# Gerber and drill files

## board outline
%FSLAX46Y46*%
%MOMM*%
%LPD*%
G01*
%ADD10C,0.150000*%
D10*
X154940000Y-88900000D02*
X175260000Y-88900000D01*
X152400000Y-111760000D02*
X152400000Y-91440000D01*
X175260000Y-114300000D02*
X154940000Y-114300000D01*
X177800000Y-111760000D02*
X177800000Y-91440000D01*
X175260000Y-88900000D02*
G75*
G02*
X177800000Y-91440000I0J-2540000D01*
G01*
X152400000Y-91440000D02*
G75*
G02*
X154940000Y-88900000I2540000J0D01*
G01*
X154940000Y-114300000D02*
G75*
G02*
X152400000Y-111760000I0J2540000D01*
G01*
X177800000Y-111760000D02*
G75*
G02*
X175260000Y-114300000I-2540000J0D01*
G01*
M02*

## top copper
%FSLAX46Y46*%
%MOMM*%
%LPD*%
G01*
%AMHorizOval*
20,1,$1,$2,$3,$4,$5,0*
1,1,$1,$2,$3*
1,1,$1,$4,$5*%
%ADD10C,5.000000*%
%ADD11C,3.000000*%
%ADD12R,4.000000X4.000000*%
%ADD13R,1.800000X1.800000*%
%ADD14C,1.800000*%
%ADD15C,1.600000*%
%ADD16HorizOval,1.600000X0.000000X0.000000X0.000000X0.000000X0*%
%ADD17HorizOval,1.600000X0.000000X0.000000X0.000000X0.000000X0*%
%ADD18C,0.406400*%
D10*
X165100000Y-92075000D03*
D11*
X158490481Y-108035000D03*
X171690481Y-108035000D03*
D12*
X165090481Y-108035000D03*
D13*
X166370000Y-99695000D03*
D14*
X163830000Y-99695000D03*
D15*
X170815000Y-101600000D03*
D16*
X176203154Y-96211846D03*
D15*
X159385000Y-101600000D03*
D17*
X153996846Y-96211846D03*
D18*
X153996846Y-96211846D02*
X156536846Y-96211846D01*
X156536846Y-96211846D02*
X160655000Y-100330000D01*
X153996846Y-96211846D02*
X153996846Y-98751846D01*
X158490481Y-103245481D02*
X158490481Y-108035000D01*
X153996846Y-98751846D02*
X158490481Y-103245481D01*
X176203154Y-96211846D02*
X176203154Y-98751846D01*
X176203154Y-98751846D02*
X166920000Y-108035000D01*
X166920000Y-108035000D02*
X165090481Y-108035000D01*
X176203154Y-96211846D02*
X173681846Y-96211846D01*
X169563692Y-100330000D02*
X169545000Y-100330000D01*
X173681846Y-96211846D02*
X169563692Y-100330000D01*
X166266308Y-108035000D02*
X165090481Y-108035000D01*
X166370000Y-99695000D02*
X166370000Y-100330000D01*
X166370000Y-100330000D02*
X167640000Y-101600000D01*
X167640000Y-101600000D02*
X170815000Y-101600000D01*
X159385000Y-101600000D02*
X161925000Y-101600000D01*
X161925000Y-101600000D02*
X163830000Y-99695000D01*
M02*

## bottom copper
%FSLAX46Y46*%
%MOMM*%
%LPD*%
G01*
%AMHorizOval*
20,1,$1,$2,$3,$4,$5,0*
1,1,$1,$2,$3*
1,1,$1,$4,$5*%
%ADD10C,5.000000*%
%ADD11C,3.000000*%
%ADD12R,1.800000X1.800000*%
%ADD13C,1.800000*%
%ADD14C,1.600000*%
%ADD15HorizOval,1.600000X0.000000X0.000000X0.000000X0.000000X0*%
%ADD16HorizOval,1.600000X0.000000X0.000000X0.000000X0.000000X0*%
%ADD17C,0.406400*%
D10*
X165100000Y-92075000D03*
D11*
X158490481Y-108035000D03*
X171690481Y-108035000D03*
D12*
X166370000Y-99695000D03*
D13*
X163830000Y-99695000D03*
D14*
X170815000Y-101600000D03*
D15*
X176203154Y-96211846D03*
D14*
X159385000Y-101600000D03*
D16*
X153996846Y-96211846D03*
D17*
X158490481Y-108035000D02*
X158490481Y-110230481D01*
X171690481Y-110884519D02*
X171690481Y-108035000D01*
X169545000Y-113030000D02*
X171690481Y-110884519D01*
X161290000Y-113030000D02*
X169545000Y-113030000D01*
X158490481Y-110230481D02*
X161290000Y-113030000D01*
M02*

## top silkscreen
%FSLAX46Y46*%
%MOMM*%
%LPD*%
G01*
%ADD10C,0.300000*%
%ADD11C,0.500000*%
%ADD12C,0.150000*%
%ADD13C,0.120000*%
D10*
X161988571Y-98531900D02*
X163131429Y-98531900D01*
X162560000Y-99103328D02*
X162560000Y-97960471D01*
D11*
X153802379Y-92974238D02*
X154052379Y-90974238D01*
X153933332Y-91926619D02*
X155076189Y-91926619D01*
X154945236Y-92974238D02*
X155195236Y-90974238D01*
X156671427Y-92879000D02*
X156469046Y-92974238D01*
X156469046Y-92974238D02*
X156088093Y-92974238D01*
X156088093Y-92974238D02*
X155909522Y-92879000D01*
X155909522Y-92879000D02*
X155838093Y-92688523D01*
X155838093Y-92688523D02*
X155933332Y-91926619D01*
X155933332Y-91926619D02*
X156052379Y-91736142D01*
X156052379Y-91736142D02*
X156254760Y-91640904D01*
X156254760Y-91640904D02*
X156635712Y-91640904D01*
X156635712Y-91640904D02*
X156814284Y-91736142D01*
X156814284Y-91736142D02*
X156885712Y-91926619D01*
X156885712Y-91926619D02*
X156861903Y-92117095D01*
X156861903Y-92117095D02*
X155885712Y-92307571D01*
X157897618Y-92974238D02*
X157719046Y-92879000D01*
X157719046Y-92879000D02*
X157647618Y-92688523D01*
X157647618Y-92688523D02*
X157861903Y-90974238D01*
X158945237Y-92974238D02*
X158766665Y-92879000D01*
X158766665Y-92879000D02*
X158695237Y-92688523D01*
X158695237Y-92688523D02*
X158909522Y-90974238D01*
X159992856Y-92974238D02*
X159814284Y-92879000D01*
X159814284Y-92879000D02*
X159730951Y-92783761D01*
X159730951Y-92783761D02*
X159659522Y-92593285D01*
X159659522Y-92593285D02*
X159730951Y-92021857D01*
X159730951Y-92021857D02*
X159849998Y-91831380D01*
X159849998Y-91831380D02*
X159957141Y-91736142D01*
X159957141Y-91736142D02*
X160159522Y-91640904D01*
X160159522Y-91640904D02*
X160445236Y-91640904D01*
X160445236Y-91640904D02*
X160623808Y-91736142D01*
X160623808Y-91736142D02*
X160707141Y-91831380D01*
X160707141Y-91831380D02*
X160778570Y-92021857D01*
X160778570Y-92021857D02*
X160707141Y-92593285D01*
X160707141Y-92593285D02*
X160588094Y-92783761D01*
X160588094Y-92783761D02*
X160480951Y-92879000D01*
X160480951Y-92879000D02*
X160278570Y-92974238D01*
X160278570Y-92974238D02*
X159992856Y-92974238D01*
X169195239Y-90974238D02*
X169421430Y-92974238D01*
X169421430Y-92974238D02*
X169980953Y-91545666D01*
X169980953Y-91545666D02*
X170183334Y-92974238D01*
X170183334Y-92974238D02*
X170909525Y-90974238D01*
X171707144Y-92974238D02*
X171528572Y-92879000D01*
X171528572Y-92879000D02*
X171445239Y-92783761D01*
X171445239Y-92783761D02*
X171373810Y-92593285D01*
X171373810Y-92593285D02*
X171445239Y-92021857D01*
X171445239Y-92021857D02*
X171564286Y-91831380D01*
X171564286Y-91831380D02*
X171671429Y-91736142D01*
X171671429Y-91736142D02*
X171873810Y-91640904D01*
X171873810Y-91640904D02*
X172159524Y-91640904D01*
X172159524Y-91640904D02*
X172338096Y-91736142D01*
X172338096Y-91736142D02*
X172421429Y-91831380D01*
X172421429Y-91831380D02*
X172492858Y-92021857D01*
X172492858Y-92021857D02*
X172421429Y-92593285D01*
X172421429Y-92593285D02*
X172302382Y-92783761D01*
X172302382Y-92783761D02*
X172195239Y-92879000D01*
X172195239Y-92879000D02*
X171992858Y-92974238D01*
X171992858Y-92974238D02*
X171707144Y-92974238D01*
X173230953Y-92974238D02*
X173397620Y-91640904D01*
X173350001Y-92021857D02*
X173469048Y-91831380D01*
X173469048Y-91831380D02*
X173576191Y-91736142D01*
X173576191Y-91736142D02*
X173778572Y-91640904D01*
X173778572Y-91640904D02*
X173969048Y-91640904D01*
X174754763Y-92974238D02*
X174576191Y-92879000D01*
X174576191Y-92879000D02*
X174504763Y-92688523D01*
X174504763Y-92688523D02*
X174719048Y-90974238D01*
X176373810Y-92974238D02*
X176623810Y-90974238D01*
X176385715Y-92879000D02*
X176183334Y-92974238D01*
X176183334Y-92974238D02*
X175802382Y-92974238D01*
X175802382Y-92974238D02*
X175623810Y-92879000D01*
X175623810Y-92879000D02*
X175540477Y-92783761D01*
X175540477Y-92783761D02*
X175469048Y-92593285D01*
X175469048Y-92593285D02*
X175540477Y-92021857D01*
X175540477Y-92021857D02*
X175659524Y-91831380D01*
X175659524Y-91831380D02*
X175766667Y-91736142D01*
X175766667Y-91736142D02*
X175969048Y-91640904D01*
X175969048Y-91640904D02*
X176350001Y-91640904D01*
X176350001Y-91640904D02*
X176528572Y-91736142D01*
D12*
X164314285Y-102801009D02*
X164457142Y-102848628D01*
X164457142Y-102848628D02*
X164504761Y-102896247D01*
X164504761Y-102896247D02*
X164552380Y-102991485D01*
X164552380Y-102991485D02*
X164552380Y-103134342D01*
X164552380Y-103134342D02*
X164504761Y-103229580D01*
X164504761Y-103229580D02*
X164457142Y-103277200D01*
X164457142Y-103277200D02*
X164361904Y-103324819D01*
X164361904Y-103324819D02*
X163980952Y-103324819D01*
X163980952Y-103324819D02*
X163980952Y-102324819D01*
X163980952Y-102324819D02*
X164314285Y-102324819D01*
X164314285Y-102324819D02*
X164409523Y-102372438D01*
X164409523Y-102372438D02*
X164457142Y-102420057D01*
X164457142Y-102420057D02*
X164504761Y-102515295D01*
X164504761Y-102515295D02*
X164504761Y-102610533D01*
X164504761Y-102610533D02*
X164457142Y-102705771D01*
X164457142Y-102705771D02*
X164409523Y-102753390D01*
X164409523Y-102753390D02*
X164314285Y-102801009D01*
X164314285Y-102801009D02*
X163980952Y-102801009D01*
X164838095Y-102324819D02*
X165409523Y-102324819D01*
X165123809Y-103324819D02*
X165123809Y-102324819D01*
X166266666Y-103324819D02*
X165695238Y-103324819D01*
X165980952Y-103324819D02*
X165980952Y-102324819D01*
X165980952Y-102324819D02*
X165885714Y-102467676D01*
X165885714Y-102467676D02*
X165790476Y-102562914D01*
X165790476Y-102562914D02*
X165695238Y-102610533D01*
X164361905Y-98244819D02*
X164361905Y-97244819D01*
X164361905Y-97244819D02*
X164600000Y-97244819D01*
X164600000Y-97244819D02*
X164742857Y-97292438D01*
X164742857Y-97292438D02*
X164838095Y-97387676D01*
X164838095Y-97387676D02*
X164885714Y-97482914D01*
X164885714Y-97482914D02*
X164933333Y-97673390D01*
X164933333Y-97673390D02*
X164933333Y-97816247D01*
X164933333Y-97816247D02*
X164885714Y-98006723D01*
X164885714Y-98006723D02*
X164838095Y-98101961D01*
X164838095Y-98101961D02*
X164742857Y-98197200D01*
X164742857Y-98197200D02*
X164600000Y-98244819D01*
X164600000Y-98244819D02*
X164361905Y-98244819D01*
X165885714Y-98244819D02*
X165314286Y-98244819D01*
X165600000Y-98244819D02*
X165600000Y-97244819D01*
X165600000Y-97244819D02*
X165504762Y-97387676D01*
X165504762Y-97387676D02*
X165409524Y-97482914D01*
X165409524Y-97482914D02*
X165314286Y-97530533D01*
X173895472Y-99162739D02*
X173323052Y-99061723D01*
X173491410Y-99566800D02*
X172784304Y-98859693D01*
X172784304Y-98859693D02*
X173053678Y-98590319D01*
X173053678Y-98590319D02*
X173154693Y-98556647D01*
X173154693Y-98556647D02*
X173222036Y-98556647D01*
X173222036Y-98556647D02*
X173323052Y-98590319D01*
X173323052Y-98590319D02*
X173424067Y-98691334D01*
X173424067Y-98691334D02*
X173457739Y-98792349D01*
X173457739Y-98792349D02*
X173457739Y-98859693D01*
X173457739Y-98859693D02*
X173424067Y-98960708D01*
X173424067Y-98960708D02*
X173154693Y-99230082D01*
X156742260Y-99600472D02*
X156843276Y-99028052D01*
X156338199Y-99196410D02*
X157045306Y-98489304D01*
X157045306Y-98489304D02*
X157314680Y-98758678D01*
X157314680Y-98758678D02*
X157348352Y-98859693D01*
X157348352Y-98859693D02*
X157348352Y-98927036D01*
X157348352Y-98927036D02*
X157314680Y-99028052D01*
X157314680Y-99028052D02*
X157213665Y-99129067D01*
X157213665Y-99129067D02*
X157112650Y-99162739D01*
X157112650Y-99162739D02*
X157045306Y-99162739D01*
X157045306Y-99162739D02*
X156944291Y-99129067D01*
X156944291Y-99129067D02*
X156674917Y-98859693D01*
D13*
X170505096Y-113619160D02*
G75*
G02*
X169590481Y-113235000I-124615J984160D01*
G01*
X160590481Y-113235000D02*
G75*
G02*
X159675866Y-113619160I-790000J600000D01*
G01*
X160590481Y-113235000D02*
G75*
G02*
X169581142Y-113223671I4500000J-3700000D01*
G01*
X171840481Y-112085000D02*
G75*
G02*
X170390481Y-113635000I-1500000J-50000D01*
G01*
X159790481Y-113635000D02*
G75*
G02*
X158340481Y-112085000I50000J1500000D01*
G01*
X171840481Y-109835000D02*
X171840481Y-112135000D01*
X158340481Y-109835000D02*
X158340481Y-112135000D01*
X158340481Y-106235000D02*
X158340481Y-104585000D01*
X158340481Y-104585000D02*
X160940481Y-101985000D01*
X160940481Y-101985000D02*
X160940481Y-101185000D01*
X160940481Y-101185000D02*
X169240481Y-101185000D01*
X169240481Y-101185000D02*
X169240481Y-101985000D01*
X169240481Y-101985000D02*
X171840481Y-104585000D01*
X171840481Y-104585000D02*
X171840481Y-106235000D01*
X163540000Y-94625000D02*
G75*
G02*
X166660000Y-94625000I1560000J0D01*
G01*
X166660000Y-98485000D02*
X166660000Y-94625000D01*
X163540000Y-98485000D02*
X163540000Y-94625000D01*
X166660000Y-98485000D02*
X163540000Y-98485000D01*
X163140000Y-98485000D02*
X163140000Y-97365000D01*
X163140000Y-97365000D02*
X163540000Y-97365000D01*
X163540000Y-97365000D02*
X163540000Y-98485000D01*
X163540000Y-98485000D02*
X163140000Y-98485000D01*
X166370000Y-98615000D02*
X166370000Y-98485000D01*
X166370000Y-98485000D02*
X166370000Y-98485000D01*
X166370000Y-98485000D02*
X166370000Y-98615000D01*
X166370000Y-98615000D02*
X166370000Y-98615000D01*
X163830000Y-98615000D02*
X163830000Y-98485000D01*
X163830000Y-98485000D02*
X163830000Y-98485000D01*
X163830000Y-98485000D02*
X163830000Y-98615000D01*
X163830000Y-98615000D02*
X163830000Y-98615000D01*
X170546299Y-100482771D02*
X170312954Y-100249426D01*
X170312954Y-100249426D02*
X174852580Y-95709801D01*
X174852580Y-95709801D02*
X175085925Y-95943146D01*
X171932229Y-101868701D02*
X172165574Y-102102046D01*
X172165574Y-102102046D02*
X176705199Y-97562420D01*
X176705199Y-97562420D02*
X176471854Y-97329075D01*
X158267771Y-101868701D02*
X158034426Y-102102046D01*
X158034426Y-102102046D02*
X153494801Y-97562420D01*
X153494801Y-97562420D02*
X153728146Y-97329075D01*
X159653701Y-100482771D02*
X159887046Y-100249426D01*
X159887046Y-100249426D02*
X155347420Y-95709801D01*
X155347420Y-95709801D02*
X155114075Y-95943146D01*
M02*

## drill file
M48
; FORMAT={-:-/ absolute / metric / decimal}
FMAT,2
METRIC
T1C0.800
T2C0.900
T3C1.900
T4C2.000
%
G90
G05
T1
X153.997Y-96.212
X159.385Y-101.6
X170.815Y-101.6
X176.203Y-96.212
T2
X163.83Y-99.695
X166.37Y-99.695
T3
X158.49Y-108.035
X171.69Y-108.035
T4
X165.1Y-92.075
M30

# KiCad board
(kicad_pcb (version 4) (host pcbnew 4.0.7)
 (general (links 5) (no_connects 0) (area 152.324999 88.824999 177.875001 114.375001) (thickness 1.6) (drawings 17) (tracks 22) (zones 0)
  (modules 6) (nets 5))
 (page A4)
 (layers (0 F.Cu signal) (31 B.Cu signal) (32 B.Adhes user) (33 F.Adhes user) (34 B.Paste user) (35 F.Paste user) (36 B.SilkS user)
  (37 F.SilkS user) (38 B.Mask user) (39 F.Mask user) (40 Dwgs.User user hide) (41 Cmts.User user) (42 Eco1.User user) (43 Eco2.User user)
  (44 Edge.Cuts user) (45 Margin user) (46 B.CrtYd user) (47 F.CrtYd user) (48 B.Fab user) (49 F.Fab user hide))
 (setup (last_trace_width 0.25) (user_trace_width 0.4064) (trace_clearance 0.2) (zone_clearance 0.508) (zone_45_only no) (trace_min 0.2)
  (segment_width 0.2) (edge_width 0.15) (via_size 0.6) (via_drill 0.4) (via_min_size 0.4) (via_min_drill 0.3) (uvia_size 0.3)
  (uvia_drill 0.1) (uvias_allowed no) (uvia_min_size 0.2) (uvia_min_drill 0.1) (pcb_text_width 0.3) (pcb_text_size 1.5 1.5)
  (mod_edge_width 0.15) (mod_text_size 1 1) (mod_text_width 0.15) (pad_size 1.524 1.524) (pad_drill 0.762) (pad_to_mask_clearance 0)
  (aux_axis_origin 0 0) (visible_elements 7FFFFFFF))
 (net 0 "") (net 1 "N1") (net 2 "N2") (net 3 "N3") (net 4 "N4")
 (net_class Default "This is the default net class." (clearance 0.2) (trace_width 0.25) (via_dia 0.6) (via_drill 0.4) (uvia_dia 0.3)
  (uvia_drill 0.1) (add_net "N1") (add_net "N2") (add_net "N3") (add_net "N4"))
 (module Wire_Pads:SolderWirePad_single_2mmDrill (layer F.Cu) (at 165.1 92.075)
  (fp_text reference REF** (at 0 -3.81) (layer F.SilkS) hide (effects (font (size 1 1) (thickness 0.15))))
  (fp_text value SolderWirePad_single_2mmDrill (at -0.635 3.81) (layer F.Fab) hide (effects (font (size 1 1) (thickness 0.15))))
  (pad 1 thru_hole circle (at 0 0) (size 5 5) (drill 2) (layers *.Cu *.Mask)))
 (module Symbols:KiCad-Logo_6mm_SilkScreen (layer B.Cu) (at 165.1 103.505 180)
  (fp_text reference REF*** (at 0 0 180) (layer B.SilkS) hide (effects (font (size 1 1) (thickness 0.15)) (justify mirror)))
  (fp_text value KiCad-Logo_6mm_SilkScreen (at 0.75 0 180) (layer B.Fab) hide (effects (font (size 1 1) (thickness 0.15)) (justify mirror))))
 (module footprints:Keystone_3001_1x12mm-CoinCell (layer F.Cu) (at 165.090481 108.035)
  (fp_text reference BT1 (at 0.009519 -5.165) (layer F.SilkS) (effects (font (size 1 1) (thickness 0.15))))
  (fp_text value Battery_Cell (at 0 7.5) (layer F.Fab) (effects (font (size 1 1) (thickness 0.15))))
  (fp_arc (start 5.29 4.6) (end 4.5 5.2) (angle -60) (layer F.SilkS) (width 0.12))
  (fp_arc (start -5.29 4.6) (end -4.5 5.2) (angle 60) (layer F.SilkS) (width 0.12))
  (fp_arc (start 0 8.9) (end -4.5 5.2) (angle 101) (layer F.SilkS) (width 0.12))
  (fp_arc (start 5.25 4.1) (end 5.3 5.6) (angle -90) (layer F.SilkS) (width 0.12))
  (fp_arc (start -5.25 4.1) (end -5.3 5.6) (angle 90) (layer F.SilkS) (width 0.12))
  (fp_line (start 6.75 1.8) (end 6.75 4.1) (layer F.SilkS) (width 0.12))
  (fp_line (start -6.75 1.8) (end -6.75 4.1) (layer F.SilkS) (width 0.12))
  (fp_line (start -6.75 -1.8) (end -6.75 -3.45) (layer F.SilkS) (width 0.12))
  (fp_line (start -6.75 -3.45) (end -4.15 -6.05) (layer F.SilkS) (width 0.12))
  (fp_line (start -4.15 -6.05) (end -4.15 -6.85) (layer F.SilkS) (width 0.12))
  (fp_line (start -4.15 -6.85) (end 4.15 -6.85) (layer F.SilkS) (width 0.12))
  (fp_line (start 4.15 -6.85) (end 4.15 -6.05) (layer F.SilkS) (width 0.12))
  (fp_line (start 4.15 -6.05) (end 6.75 -3.45) (layer F.SilkS) (width 0.12))
  (fp_line (start 6.75 -3.45) (end 6.75 -1.8) (layer F.SilkS) (width 0.12))
  (pad 1 thru_hole circle (at -6.6 0) (size 3 3) (drill 1.9) (layers *.Cu *.Mask) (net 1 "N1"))
  (pad 1 thru_hole circle (at 6.6 0) (size 3 3) (drill 1.9) (layers *.Cu *.Mask) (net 1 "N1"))
  (pad 2 smd rect (at 0 0) (size 4 4) (layers F.Cu F.Mask) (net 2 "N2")))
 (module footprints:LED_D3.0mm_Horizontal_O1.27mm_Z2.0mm (layer F.Cu) (at 166.37 99.695 180)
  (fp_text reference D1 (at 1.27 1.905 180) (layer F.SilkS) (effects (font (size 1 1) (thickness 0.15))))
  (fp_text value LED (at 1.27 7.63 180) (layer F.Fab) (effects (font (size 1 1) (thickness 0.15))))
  (fp_arc (start 1.27 5.07) (end -0.29 5.07) (angle -180) (layer F.SilkS) (width 0.12))
  (fp_line (start -0.29 1.21) (end -0.29 5.07) (layer F.SilkS) (width 0.12))
  (fp_line (start 2.83 1.21) (end 2.83 5.07) (layer F.SilkS) (width 0.12))
  (fp_line (start -0.29 1.21) (end 2.83 1.21) (layer F.SilkS) (width 0.12))
  (fp_line (start 3.23 1.21) (end 3.23 2.33) (layer F.SilkS) (width 0.12))
  (fp_line (start 3.23 2.33) (end 2.83 2.33) (layer F.SilkS) (width 0.12))
  (fp_line (start 2.83 2.33) (end 2.83 1.21) (layer F.SilkS) (width 0.12))
  (fp_line (start 2.83 1.21) (end 3.23 1.21) (layer F.SilkS) (width 0.12))
  (fp_line (start 0 1.08) (end 0 1.21) (layer F.SilkS) (width 0.12))
  (fp_line (start 0 1.21) (end 0 1.21) (layer F.SilkS) (width 0.12))
  (fp_line (start 0 1.21) (end 0 1.08) (layer F.SilkS) (width 0.12))
  (fp_line (start 0 1.08) (end 0 1.08) (layer F.SilkS) (width 0.12))
  (fp_line (start 2.54 1.08) (end 2.54 1.21) (layer F.SilkS) (width 0.12))
  (fp_line (start 2.54 1.21) (end 2.54 1.21) (layer F.SilkS) (width 0.12))
  (fp_line (start 2.54 1.21) (end 2.54 1.08) (layer F.SilkS) (width 0.12))
  (fp_line (start 2.54 1.08) (end 2.54 1.08) (layer F.SilkS) (width 0.12))
  (pad 1 thru_hole rect (at 0 0 180) (size 1.8 1.8) (drill 0.9) (layers *.Cu *.Mask) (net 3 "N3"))
  (pad 2 thru_hole circle (at 2.54 0 180) (size 1.8 1.8) (drill 0.9) (layers *.Cu *.Mask) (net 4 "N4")))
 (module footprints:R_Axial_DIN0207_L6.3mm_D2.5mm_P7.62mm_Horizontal (layer F.Cu) (at 170.815 101.6 45)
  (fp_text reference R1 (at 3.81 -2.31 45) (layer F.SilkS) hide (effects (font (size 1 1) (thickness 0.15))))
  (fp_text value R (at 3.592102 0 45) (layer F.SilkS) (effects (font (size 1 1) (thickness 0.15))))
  (fp_line (start 0.6 -0.98) (end 0.6 -1.31) (layer F.SilkS) (width 0.12))
  (fp_line (start 0.6 -1.31) (end 7.02 -1.31) (layer F.SilkS) (width 0.12))
  (fp_line (start 7.02 -1.31) (end 7.02 -0.98) (layer F.SilkS) (width 0.12))
  (fp_line (start 0.6 0.98) (end 0.6 1.31) (layer F.SilkS) (width 0.12))
  (fp_line (start 0.6 1.31) (end 7.02 1.31) (layer F.SilkS) (width 0.12))
  (fp_line (start 7.02 1.31) (end 7.02 0.98) (layer F.SilkS) (width 0.12))
  (pad 1 thru_hole circle (at 0 0 45) (size 1.6 1.6) (drill 0.8) (layers *.Cu *.Mask) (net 3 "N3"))
  (pad 2 thru_hole oval (at 7.62 0 45) (size 1.6 1.6) (drill 0.8) (layers *.Cu *.Mask) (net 2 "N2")))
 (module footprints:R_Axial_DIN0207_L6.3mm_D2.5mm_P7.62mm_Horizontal (layer F.Cu) (at 159.385 101.6 135)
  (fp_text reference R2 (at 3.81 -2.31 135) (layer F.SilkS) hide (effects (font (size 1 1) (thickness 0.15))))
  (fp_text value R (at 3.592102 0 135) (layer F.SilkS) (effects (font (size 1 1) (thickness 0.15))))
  (fp_line (start 0.6 -0.98) (end 0.6 -1.31) (layer F.SilkS) (width 0.12))
  (fp_line (start 0.6 -1.31) (end 7.02 -1.31) (layer F.SilkS) (width 0.12))
  (fp_line (start 7.02 -1.31) (end 7.02 -0.98) (layer F.SilkS) (width 0.12))
  (fp_line (start 0.6 0.98) (end 0.6 1.31) (layer F.SilkS) (width 0.12))
  (fp_line (start 0.6 1.31) (end 7.02 1.31) (layer F.SilkS) (width 0.12))
  (fp_line (start 7.02 1.31) (end 7.02 0.98) (layer F.SilkS) (width 0.12))
  (pad 1 thru_hole circle (at 0 0 135) (size 1.6 1.6) (drill 0.8) (layers *.Cu *.Mask) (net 4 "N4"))
  (pad 2 thru_hole oval (at 7.62 0 135) (size 1.6 1.6) (drill 0.8) (layers *.Cu *.Mask) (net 1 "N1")))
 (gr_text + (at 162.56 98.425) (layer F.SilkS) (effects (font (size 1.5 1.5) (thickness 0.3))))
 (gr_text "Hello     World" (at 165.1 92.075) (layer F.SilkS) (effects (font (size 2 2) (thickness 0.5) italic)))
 (gr_line (start 154.94 88.9) (end 175.26 88.9) (angle 90) (layer Edge.Cuts) (width 0.15))
 (gr_line (start 152.4 111.76) (end 152.4 91.44) (angle 90) (layer Edge.Cuts) (width 0.15))
 (gr_line (start 175.26 114.3) (end 154.94 114.3) (angle 90) (layer Edge.Cuts) (width 0.15))
 (gr_line (start 177.8 111.76) (end 177.8 91.44) (angle 90) (layer Edge.Cuts) (width 0.15))
 (gr_arc (start 175.26 91.44) (end 175.26 88.9) (angle 90) (layer Edge.Cuts) (width 0.15))
 (gr_arc (start 154.94 91.44) (end 152.4 91.44) (angle 90) (layer Edge.Cuts) (width 0.15))
 (gr_arc (start 154.94 111.76) (end 154.94 114.3) (angle 90) (layer Edge.Cuts) (width 0.15))
 (gr_arc (start 175.26 111.76) (end 177.8 111.76) (angle 90) (layer Edge.Cuts) (width 0.15))
 (segment (start 153.996846 96.211846) (end 156.536846 96.211846) (width 0.4064) (layer F.Cu) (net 1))
 (segment (start 156.536846 96.211846) (end 160.655 100.33) (width 0.4064) (layer F.Cu) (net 1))
 (segment (start 158.490481 108.035) (end 158.490481 110.230481) (width 0.4064) (layer B.Cu) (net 1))
 (segment (start 171.690481 110.884519) (end 171.690481 108.035) (width 0.4064) (layer B.Cu) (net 1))
 (segment (start 169.545 113.03) (end 171.690481 110.884519) (width 0.4064) (layer B.Cu) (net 1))
 (segment (start 161.29 113.03) (end 169.545 113.03) (width 0.4064) (layer B.Cu) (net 1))
 (segment (start 158.490481 110.230481) (end 161.29 113.03) (width 0.4064) (layer B.Cu) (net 1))
 (segment (start 153.996846 96.211846) (end 153.996846 98.751846) (width 0.4064) (layer F.Cu) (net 1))
 (segment (start 158.490481 103.245481) (end 158.490481 108.035) (width 0.4064) (layer F.Cu) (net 1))
 (segment (start 153.996846 98.751846) (end 158.490481 103.245481) (width 0.4064) (layer F.Cu) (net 1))
 (segment (start 176.203154 96.211846) (end 176.203154 98.751846) (width 0.4064) (layer F.Cu) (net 2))
 (segment (start 176.203154 98.751846) (end 166.92 108.035) (width 0.4064) (layer F.Cu) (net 2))
 (segment (start 166.92 108.035) (end 165.090481 108.035) (width 0.4064) (layer F.Cu) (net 2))
 (segment (start 176.203154 96.211846) (end 173.681846 96.211846) (width 0.4064) (layer F.Cu) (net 2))
 (segment (start 169.563692 100.33) (end 169.545 100.33) (width 0.4064) (layer F.Cu) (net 2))
 (segment (start 173.681846 96.211846) (end 169.563692 100.33) (width 0.4064) (layer F.Cu) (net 2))
 (segment (start 166.266308 108.035) (end 165.090481 108.035) (width 0.4064) (layer F.Cu) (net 2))
 (segment (start 166.37 99.695) (end 166.37 100.33) (width 0.4064) (layer F.Cu) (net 3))
 (segment (start 166.37 100.33) (end 167.64 101.6) (width 0.4064) (layer F.Cu) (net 3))
 (segment (start 167.64 101.6) (end 170.815 101.6) (width 0.4064) (layer F.Cu) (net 3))
 (segment (start 159.385 101.6) (end 161.925 101.6) (width 0.4064) (layer F.Cu) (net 4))
 (segment (start 161.925 101.6) (end 163.83 99.695) (width 0.4064) (layer F.Cu) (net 4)))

